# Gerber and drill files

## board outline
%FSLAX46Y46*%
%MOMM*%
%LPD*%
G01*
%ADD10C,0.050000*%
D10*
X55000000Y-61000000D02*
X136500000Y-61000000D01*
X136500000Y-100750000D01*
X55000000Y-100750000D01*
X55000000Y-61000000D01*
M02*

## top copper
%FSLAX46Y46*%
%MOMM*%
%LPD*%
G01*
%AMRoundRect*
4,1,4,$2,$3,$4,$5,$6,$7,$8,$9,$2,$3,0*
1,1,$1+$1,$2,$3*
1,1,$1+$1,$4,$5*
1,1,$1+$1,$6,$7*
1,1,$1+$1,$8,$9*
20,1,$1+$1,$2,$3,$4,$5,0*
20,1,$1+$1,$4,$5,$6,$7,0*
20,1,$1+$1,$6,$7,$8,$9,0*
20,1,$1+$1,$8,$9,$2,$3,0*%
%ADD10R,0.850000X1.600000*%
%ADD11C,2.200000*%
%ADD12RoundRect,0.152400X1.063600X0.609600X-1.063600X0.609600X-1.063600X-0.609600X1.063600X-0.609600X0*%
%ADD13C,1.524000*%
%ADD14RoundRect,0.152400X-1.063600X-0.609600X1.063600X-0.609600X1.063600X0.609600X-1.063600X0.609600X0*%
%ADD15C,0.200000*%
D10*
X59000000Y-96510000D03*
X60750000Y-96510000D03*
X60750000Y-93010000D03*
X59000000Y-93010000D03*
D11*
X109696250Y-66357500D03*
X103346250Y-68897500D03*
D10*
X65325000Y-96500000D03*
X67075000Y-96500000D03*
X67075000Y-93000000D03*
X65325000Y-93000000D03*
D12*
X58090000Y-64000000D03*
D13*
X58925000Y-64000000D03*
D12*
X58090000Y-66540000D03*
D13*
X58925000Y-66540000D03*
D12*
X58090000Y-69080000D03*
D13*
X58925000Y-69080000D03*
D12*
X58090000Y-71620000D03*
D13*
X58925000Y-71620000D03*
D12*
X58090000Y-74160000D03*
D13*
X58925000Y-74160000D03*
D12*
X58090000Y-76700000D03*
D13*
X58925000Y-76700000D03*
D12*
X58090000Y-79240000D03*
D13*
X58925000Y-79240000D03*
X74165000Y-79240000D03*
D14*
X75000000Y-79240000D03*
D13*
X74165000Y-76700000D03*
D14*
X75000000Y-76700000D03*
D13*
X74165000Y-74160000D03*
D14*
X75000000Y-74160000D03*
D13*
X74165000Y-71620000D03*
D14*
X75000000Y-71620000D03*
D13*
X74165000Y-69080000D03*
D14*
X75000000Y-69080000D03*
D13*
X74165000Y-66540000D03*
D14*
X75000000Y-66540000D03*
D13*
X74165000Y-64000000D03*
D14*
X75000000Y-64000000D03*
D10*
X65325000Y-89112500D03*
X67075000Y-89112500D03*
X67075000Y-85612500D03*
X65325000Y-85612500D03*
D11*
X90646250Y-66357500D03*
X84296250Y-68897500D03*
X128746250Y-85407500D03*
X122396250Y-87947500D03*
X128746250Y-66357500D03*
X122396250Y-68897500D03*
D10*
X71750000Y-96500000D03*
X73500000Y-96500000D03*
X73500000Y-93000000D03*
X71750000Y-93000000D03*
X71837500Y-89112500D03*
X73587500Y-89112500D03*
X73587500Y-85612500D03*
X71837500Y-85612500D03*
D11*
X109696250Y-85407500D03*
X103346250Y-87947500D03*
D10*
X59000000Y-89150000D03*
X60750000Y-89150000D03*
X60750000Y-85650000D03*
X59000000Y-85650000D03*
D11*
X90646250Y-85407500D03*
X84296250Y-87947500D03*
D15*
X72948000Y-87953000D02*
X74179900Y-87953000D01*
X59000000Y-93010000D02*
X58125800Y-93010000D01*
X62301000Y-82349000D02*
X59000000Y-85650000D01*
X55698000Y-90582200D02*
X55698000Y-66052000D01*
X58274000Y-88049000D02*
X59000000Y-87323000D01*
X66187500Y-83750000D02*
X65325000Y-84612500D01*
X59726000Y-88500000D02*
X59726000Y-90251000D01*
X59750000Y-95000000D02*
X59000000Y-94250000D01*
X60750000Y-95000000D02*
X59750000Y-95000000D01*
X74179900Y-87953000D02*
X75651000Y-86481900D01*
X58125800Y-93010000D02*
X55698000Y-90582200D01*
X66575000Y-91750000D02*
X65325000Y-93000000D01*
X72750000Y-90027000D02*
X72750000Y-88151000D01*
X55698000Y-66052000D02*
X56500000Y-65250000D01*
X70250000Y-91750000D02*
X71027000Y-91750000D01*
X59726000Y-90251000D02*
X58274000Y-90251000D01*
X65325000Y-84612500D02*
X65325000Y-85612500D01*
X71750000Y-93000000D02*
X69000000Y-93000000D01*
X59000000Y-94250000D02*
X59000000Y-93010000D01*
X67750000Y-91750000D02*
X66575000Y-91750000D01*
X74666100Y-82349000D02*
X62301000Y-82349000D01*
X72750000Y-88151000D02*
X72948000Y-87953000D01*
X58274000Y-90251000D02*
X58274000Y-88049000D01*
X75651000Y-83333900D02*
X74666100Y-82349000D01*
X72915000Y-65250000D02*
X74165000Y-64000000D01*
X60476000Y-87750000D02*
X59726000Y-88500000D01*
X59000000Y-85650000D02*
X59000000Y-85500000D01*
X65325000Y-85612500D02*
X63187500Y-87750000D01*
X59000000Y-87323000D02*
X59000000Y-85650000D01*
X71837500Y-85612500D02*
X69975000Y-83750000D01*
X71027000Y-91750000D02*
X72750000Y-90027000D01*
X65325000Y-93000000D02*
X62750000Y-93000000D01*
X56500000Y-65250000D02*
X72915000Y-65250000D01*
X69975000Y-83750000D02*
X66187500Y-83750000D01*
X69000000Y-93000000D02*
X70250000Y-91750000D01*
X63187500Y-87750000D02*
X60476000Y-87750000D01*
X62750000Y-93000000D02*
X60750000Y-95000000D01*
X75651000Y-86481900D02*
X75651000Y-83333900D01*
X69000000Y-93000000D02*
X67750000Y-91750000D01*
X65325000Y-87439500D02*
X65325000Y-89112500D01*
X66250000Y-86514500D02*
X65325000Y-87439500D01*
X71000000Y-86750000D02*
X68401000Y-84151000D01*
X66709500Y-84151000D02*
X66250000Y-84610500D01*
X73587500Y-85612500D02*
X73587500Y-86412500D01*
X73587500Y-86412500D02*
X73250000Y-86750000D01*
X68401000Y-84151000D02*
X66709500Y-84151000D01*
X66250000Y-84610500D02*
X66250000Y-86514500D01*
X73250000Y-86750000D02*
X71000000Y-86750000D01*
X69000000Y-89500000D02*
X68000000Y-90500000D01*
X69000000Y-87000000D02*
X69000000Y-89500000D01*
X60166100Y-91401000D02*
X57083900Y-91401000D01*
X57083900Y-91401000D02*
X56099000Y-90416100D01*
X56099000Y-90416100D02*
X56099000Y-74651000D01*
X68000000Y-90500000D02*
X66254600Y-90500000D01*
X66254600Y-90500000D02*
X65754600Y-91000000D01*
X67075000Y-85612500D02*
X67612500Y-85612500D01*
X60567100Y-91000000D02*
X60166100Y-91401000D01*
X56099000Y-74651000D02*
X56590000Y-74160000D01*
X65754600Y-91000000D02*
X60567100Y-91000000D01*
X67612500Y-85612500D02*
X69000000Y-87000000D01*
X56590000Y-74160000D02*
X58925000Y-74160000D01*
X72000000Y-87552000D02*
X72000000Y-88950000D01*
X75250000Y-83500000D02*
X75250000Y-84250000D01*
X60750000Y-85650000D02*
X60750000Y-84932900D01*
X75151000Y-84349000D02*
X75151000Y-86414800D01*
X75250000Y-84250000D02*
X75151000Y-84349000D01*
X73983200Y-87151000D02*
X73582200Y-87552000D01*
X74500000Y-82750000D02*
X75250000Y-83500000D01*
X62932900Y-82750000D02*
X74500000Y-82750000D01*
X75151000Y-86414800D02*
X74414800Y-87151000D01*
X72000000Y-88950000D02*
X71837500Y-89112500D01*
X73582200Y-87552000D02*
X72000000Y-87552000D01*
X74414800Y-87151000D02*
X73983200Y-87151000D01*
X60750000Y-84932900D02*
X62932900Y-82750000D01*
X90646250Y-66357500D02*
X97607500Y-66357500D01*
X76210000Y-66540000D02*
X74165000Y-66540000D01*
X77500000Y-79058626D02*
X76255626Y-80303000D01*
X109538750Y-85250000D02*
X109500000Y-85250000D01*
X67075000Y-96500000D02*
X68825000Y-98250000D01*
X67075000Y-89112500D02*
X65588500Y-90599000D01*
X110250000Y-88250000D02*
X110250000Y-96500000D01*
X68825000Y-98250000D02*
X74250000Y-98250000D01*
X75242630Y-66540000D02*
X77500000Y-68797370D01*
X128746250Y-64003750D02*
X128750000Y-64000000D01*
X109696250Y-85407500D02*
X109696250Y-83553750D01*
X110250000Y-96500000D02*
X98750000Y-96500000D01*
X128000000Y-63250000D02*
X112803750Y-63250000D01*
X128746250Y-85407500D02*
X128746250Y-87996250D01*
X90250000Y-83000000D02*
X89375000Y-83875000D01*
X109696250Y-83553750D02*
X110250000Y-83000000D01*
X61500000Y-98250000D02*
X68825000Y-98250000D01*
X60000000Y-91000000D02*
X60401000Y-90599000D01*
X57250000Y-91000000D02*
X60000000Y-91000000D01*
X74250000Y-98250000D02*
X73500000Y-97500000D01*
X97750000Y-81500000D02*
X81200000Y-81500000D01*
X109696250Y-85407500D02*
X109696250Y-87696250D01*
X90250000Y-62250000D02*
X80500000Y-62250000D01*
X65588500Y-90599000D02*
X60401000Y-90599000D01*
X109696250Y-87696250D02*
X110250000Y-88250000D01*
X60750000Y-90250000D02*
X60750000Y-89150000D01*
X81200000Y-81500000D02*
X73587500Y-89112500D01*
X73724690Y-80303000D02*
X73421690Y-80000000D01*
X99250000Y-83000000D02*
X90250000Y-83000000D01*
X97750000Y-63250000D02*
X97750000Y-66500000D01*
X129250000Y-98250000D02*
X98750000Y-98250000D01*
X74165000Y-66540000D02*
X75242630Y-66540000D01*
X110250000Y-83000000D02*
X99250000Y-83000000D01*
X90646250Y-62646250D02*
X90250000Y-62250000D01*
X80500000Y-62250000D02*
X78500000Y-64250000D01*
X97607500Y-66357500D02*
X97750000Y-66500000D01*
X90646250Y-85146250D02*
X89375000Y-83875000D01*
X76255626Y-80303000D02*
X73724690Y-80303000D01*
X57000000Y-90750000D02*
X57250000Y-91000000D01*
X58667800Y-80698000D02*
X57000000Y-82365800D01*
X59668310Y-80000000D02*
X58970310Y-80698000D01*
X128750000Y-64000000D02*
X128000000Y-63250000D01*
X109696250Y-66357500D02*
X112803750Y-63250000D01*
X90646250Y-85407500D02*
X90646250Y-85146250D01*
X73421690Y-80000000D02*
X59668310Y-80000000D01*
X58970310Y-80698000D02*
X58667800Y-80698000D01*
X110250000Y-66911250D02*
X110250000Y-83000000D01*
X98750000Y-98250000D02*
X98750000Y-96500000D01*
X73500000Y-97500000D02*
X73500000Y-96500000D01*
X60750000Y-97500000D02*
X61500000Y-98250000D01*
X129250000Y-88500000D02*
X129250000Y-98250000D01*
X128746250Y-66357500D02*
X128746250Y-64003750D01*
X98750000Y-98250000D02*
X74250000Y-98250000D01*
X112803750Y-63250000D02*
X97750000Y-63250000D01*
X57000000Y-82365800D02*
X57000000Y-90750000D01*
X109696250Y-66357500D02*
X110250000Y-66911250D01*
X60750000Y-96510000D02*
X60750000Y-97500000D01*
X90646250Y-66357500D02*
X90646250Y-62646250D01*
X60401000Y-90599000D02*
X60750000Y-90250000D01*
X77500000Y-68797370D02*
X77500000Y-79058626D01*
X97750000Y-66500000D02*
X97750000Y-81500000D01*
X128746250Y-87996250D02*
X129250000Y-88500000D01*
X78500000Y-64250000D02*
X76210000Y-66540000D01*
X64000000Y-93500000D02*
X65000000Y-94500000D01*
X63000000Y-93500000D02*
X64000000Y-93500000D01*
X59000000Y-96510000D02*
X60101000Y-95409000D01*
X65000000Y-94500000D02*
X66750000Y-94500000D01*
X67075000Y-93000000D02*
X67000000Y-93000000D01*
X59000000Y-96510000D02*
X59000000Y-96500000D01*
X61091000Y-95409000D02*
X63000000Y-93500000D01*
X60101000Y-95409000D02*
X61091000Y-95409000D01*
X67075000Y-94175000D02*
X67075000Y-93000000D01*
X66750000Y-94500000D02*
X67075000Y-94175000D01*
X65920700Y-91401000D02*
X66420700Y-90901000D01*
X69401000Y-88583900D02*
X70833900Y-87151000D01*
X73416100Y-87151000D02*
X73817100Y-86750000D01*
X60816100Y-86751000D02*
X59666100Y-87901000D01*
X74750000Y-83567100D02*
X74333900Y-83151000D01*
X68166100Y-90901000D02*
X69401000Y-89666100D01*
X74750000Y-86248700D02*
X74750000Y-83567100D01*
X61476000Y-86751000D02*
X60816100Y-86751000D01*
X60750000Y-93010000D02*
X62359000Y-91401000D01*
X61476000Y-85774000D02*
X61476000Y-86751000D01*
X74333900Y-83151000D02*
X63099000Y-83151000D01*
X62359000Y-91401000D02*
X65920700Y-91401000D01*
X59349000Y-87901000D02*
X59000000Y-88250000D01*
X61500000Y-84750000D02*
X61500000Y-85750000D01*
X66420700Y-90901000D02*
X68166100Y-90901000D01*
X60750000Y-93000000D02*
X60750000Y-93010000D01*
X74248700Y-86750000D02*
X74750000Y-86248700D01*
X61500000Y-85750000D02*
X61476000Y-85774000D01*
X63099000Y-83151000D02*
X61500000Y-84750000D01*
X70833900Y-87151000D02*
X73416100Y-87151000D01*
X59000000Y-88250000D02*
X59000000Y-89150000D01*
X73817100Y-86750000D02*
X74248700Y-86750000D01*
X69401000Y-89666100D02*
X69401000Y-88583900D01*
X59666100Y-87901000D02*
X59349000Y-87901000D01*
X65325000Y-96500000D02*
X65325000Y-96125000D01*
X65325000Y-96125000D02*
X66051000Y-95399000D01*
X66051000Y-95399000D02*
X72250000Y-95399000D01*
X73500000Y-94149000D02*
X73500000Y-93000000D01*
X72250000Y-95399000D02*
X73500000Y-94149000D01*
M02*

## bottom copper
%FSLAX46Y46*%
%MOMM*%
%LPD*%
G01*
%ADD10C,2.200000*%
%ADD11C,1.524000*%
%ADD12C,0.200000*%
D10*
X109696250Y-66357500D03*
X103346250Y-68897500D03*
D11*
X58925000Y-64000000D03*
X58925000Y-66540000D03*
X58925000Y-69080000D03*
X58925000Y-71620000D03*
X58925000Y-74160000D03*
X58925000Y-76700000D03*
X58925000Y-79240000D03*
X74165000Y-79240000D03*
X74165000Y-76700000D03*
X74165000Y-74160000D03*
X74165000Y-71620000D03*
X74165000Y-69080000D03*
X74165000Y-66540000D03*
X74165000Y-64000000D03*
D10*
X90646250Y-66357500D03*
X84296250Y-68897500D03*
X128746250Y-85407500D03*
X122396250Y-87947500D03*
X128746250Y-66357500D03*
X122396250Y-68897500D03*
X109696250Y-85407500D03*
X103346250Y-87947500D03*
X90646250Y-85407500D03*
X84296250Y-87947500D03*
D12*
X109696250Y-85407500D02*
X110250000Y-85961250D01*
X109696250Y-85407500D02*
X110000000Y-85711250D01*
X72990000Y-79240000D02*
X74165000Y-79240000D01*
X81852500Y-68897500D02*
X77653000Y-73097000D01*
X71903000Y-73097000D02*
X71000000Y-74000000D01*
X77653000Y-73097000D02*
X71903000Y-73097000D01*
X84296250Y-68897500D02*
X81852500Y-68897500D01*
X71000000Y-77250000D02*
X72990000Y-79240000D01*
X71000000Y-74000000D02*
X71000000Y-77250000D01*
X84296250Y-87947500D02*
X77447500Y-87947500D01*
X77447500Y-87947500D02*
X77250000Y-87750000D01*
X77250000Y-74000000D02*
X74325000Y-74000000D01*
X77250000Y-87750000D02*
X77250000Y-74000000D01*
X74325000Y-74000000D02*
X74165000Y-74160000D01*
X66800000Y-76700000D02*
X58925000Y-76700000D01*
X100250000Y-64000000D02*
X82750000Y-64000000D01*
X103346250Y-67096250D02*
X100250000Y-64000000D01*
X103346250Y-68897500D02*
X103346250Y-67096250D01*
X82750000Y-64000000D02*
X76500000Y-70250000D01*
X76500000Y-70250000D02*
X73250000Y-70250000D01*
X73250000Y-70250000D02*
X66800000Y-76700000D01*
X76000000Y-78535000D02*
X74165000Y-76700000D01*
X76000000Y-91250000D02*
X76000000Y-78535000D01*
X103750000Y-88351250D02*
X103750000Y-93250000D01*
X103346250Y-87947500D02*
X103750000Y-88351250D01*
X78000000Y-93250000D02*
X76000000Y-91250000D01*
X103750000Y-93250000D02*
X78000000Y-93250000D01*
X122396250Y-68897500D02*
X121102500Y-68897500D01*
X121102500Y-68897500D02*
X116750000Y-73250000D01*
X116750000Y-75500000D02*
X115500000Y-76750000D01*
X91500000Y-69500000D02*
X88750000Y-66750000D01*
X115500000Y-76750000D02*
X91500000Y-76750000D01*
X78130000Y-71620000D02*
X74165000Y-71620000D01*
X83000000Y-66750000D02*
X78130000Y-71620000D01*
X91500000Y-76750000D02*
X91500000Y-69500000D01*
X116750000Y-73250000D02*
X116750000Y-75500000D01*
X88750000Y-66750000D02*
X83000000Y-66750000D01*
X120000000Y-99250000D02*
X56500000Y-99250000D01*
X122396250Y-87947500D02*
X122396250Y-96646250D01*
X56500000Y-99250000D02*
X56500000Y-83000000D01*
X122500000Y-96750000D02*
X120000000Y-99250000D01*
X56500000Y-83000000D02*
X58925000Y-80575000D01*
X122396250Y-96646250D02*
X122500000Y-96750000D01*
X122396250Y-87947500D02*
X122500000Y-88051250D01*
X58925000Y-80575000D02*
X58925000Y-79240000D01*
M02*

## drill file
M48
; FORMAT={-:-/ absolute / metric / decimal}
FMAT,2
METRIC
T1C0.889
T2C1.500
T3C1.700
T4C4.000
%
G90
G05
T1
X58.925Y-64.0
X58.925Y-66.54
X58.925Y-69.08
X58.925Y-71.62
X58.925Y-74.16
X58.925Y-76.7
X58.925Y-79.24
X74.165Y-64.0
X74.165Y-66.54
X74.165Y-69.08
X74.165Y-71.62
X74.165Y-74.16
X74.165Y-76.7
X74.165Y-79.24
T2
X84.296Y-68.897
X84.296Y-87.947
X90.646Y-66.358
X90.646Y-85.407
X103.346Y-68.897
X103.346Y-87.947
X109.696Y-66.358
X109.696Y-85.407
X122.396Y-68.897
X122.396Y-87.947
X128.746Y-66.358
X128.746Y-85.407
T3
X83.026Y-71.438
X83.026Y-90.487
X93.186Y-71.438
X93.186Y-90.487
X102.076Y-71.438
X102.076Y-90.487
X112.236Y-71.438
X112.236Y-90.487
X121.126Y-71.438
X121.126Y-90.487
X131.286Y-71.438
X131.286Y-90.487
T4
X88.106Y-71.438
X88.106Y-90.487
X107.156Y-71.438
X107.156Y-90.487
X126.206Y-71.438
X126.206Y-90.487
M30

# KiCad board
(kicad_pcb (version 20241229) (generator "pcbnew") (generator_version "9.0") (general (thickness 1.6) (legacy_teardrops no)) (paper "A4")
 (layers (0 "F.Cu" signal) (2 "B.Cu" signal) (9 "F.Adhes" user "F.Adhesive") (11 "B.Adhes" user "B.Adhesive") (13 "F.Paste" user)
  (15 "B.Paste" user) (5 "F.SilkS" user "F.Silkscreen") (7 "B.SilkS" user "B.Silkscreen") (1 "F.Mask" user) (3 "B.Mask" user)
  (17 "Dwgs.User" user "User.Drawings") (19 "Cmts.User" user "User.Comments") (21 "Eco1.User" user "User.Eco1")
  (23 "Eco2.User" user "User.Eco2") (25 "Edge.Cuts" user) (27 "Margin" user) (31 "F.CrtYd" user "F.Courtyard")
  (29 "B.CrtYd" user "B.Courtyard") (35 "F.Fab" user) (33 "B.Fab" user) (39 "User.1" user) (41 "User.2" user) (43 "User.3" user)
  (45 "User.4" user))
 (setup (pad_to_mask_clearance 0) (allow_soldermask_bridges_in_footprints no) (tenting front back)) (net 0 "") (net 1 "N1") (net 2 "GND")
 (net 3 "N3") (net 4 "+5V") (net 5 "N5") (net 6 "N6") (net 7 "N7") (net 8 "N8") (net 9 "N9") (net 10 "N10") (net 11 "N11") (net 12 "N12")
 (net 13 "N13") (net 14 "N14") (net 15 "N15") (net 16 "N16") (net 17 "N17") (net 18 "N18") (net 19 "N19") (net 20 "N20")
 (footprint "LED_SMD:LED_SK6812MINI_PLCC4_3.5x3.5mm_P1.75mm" (layer "F.Cu") (at 59.875 94.76 90)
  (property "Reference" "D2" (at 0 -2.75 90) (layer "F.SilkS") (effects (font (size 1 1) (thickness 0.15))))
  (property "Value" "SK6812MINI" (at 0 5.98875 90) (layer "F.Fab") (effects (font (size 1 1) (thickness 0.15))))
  (pad "1" smd rect (at -1.75 -0.875 90) (size 1.6 0.85) (layers "F.Cu" "F.Mask" "F.Paste") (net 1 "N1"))
  (pad "2" smd rect (at -1.75 0.875 90) (size 1.6 0.85) (layers "F.Cu" "F.Mask" "F.Paste") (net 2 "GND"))
  (pad "3" smd rect (at 1.75 0.875 90) (size 1.6 0.85) (layers "F.Cu" "F.Mask" "F.Paste") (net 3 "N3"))
  (pad "4" smd rect (at 1.75 -0.875 90) (size 1.6 0.85) (layers "F.Cu" "F.Mask" "F.Paste") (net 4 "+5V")))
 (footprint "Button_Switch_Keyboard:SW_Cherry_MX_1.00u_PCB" (layer "F.Cu") (at 109.69625 66.3575)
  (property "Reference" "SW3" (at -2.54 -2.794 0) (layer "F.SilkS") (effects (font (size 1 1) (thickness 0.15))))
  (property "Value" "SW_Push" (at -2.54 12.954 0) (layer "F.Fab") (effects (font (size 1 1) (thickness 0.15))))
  (pad "" np_thru_hole circle (at -7.62 5.08) (size 1.7 1.7) (drill 1.7) (layers "*.Cu" "*.Mask"))
  (pad "" np_thru_hole circle (at -2.54 5.08) (size 4 4) (drill 4) (layers "*.Cu" "*.Mask"))
  (pad "" np_thru_hole circle (at 2.54 5.08) (size 1.7 1.7) (drill 1.7) (layers "*.Cu" "*.Mask"))
  (pad "1" thru_hole circle (at 0 0) (size 2.2 2.2) (drill 1.5) (layers "*.Cu" "*.Mask") (remove_unused_layers no) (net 2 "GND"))
  (pad "2" thru_hole circle (at -6.35 2.54) (size 2.2 2.2) (drill 1.5) (layers "*.Cu" "*.Mask") (remove_unused_layers no) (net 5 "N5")))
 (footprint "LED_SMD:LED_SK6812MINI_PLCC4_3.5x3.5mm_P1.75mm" (layer "F.Cu") (at 66.2 94.75 90)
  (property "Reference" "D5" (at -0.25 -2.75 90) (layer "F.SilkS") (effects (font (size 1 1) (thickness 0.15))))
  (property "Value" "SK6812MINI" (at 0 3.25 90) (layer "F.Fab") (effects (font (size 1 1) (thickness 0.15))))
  (pad "1" smd rect (at -1.75 -0.875 90) (size 1.6 0.85) (layers "F.Cu" "F.Mask" "F.Paste") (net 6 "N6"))
  (pad "2" smd rect (at -1.75 0.875 90) (size 1.6 0.85) (layers "F.Cu" "F.Mask" "F.Paste") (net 2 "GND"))
  (pad "3" smd rect (at 1.75 0.875 90) (size 1.6 0.85) (layers "F.Cu" "F.Mask" "F.Paste") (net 1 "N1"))
  (pad "4" smd rect (at 1.75 -0.875 90) (size 1.6 0.85) (layers "F.Cu" "F.Mask" "F.Paste") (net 4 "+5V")))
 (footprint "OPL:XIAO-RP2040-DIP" (layer "F.Cu") (at 66.545 71.62)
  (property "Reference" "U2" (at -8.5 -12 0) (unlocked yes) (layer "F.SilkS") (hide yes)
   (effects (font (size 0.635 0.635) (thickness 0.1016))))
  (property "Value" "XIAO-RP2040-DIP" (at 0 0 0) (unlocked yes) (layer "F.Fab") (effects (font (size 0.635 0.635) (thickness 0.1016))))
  (pad "1" smd roundrect (at -8.455 -7.62 180) (size 2.432 1.524) (layers "F.Cu" "F.Mask") (roundrect_rratio 0.1) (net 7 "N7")
   (thermal_bridge_angle 45))
  (pad "1" thru_hole circle (at -7.62 -7.62 180) (size 1.524 1.524) (drill 0.889) (layers "*.Cu" "*.Mask") (remove_unused_layers no)
   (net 7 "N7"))
  (pad "2" smd roundrect (at -8.455 -5.08 180) (size 2.432 1.524) (layers "F.Cu" "F.Mask") (roundrect_rratio 0.1) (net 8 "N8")
   (thermal_bridge_angle 45))
  (pad "2" thru_hole circle (at -7.62 -5.08 180) (size 1.524 1.524) (drill 0.889) (layers "*.Cu" "*.Mask") (remove_unused_layers no)
   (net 8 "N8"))
  (pad "3" smd roundrect (at -8.455 -2.54 180) (size 2.432 1.524) (layers "F.Cu" "F.Mask") (roundrect_rratio 0.1) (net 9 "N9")
   (thermal_bridge_angle 45))
  (pad "3" thru_hole circle (at -7.62 -2.54 180) (size 1.524 1.524) (drill 0.889) (layers "*.Cu" "*.Mask") (remove_unused_layers no)
   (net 9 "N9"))
  (pad "4" smd roundrect (at -8.455 0 180) (size 2.432 1.524) (layers "F.Cu" "F.Mask") (roundrect_rratio 0.1) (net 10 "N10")
   (thermal_bridge_angle 45))
  (pad "4" thru_hole circle (at -7.62 0 180) (size 1.524 1.524) (drill 0.889) (layers "*.Cu" "*.Mask") (remove_unused_layers no)
   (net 10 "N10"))
  (pad "5" smd roundrect (at -8.455 2.54 180) (size 2.432 1.524) (layers "F.Cu" "F.Mask") (roundrect_rratio 0.1) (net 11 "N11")
   (thermal_bridge_angle 45))
  (pad "5" thru_hole circle (at -7.62 2.54 180) (size 1.524 1.524) (drill 0.889) (layers "*.Cu" "*.Mask") (remove_unused_layers no)
   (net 11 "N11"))
  (pad "6" smd roundrect (at -8.455 5.08 180) (size 2.432 1.524) (layers "F.Cu" "F.Mask") (roundrect_rratio 0.1) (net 5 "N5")
   (thermal_bridge_angle 45))
  (pad "6" thru_hole circle (at -7.62 5.08 180) (size 1.524 1.524) (drill 0.889) (layers "*.Cu" "*.Mask") (remove_unused_layers no)
   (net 5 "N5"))
  (pad "7" smd roundrect (at -8.455 7.62 180) (size 2.432 1.524) (layers "F.Cu" "F.Mask") (roundrect_rratio 0.1) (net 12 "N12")
   (thermal_bridge_angle 45))
  (pad "7" thru_hole circle (at -7.62 7.62 180) (size 1.524 1.524) (drill 0.889) (layers "*.Cu" "*.Mask") (remove_unused_layers no)
   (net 12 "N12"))
  (pad "8" thru_hole circle (at 7.62 7.62) (size 1.524 1.524) (drill 0.889) (layers "*.Cu" "*.Mask") (remove_unused_layers no)
   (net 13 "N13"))
  (pad "8" smd roundrect (at 8.455 7.62) (size 2.432 1.524) (layers "F.Cu" "F.Mask") (roundrect_rratio 0.1) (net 13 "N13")
   (thermal_bridge_angle 45))
  (pad "9" thru_hole circle (at 7.62 5.08) (size 1.524 1.524) (drill 0.889) (layers "*.Cu" "*.Mask") (remove_unused_layers no)
   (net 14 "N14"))
  (pad "9" smd roundrect (at 8.455 5.08) (size 2.432 1.524) (layers "F.Cu" "F.Mask") (roundrect_rratio 0.1) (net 14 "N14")
   (thermal_bridge_angle 45))
  (pad "10" thru_hole circle (at 7.62 2.54) (size 1.524 1.524) (drill 0.889) (layers "*.Cu" "*.Mask") (remove_unused_layers no)
   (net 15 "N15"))
  (pad "10" smd roundrect (at 8.455 2.54) (size 2.432 1.524) (layers "F.Cu" "F.Mask") (roundrect_rratio 0.1) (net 15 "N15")
   (thermal_bridge_angle 45))
  (pad "11" thru_hole circle (at 7.62 0) (size 1.524 1.524) (drill 0.889) (layers "*.Cu" "*.Mask") (remove_unused_layers no) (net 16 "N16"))
  (pad "11" smd roundrect (at 8.455 0) (size 2.432 1.524) (layers "F.Cu" "F.Mask") (roundrect_rratio 0.1) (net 16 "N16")
   (thermal_bridge_angle 45))
  (pad "12" thru_hole circle (at 7.62 -2.54) (size 1.524 1.524) (drill 0.889) (layers "*.Cu" "*.Mask") (remove_unused_layers no)
   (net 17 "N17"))
  (pad "12" smd roundrect (at 8.455 -2.54) (size 2.432 1.524) (layers "F.Cu" "F.Mask") (roundrect_rratio 0.1) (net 17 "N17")
   (thermal_bridge_angle 45))
  (pad "13" thru_hole circle (at 7.62 -5.08) (size 1.524 1.524) (drill 0.889) (layers "*.Cu" "*.Mask") (remove_unused_layers no)
   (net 2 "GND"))
  (pad "13" smd roundrect (at 8.455 -5.08) (size 2.432 1.524) (layers "F.Cu" "F.Mask") (roundrect_rratio 0.1) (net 2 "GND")
   (thermal_bridge_angle 45))
  (pad "14" thru_hole circle (at 7.62 -7.62) (size 1.524 1.524) (drill 0.889) (layers "*.Cu" "*.Mask") (remove_unused_layers no)
   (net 4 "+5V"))
  (pad "14" smd roundrect (at 8.455 -7.62) (size 2.432 1.524) (layers "F.Cu" "F.Mask") (roundrect_rratio 0.1) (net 4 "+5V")
   (thermal_bridge_angle 45)))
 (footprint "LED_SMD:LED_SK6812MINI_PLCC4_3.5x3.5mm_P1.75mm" (layer "F.Cu") (at 66.2 87.3625 90)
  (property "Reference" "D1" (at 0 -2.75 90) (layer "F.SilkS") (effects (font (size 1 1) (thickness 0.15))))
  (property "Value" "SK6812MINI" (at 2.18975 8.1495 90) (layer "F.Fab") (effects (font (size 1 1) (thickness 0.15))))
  (pad "1" smd rect (at -1.75 -0.875 90) (size 1.6 0.85) (layers "F.Cu" "F.Mask" "F.Paste") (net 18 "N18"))
  (pad "2" smd rect (at -1.75 0.875 90) (size 1.6 0.85) (layers "F.Cu" "F.Mask" "F.Paste") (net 2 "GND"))
  (pad "3" smd rect (at 1.75 0.875 90) (size 1.6 0.85) (layers "F.Cu" "F.Mask" "F.Paste") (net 11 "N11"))
  (pad "4" smd rect (at 1.75 -0.875 90) (size 1.6 0.85) (layers "F.Cu" "F.Mask" "F.Paste") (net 4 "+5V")))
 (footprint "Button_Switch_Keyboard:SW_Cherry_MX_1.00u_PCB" (layer "F.Cu") (at 90.64625 66.3575)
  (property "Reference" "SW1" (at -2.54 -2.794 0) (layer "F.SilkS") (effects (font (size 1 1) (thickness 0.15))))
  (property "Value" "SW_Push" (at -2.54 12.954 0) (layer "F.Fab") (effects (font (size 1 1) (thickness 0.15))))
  (pad "" np_thru_hole circle (at -7.62 5.08) (size 1.7 1.7) (drill 1.7) (layers "*.Cu" "*.Mask"))
  (pad "" np_thru_hole circle (at -2.54 5.08) (size 4 4) (drill 4) (layers "*.Cu" "*.Mask"))
  (pad "" np_thru_hole circle (at 2.54 5.08) (size 1.7 1.7) (drill 1.7) (layers "*.Cu" "*.Mask"))
  (pad "1" thru_hole circle (at 0 0) (size 2.2 2.2) (drill 1.5) (layers "*.Cu" "*.Mask") (remove_unused_layers no) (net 2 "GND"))
  (pad "2" thru_hole circle (at -6.35 2.54) (size 2.2 2.2) (drill 1.5) (layers "*.Cu" "*.Mask") (remove_unused_layers no) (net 13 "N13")))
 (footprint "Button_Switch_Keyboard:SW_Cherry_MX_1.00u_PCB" (layer "F.Cu") (at 128.74625 85.4075)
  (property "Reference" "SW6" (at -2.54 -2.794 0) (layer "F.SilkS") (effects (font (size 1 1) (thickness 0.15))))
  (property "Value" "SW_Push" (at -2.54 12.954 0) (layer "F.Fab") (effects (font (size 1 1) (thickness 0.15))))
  (pad "" np_thru_hole circle (at -7.62 5.08) (size 1.7 1.7) (drill 1.7) (layers "*.Cu" "*.Mask"))
  (pad "" np_thru_hole circle (at -2.54 5.08) (size 4 4) (drill 4) (layers "*.Cu" "*.Mask"))
  (pad "" np_thru_hole circle (at 2.54 5.08) (size 1.7 1.7) (drill 1.7) (layers "*.Cu" "*.Mask"))
  (pad "1" thru_hole circle (at 0 0) (size 2.2 2.2) (drill 1.5) (layers "*.Cu" "*.Mask") (remove_unused_layers no) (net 2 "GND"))
  (pad "2" thru_hole circle (at -6.35 2.54) (size 2.2 2.2) (drill 1.5) (layers "*.Cu" "*.Mask") (remove_unused_layers no) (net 12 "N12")))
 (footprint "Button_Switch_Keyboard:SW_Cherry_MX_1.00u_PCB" (layer "F.Cu") (at 128.74625 66.3575)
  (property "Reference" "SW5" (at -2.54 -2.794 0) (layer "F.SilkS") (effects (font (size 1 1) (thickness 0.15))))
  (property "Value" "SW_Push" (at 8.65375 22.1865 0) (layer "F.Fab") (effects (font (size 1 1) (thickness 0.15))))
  (pad "" np_thru_hole circle (at -7.62 5.08) (size 1.7 1.7) (drill 1.7) (layers "*.Cu" "*.Mask"))
  (pad "" np_thru_hole circle (at -2.54 5.08) (size 4 4) (drill 4) (layers "*.Cu" "*.Mask"))
  (pad "" np_thru_hole circle (at 2.54 5.08) (size 1.7 1.7) (drill 1.7) (layers "*.Cu" "*.Mask"))
  (pad "1" thru_hole circle (at 0 0) (size 2.2 2.2) (drill 1.5) (layers "*.Cu" "*.Mask") (remove_unused_layers no) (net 2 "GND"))
  (pad "2" thru_hole circle (at -6.35 2.54) (size 2.2 2.2) (drill 1.5) (layers "*.Cu" "*.Mask") (remove_unused_layers no) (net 16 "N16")))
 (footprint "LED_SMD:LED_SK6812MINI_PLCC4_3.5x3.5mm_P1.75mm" (layer "F.Cu") (at 72.625 94.75 90)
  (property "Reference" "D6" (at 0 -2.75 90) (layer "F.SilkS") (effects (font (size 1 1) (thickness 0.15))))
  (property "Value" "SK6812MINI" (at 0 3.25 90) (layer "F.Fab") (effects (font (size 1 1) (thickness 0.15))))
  (pad "1" smd rect (at -1.75 -0.875 90) (size 1.6 0.85) (layers "F.Cu" "F.Mask" "F.Paste") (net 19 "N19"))
  (pad "2" smd rect (at -1.75 0.875 90) (size 1.6 0.85) (layers "F.Cu" "F.Mask" "F.Paste") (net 2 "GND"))
  (pad "3" smd rect (at 1.75 0.875 90) (size 1.6 0.85) (layers "F.Cu" "F.Mask" "F.Paste") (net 6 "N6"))
  (pad "4" smd rect (at 1.75 -0.875 90) (size 1.6 0.85) (layers "F.Cu" "F.Mask" "F.Paste") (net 4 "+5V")))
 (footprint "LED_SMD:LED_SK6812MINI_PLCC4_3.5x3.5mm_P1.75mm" (layer "F.Cu") (at 72.7125 87.3625 90)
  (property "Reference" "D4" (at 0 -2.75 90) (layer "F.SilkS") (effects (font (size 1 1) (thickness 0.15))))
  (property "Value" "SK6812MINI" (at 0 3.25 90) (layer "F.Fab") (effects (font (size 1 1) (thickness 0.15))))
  (pad "1" smd rect (at -1.75 -0.875 90) (size 1.6 0.85) (layers "F.Cu" "F.Mask" "F.Paste") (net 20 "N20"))
  (pad "2" smd rect (at -1.75 0.875 90) (size 1.6 0.85) (layers "F.Cu" "F.Mask" "F.Paste") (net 2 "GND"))
  (pad "3" smd rect (at 1.75 0.875 90) (size 1.6 0.85) (layers "F.Cu" "F.Mask" "F.Paste") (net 18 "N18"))
  (pad "4" smd rect (at 1.75 -0.875 90) (size 1.6 0.85) (layers "F.Cu" "F.Mask" "F.Paste") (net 4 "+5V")))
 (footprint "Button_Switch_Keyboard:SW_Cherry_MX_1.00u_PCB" (layer "F.Cu") (at 109.69625 85.4075)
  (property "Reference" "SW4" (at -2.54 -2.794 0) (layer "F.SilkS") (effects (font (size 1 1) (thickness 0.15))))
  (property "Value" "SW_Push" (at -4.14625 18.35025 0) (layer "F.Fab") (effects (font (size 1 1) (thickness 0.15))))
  (pad "" np_thru_hole circle (at -7.62 5.08) (size 1.7 1.7) (drill 1.7) (layers "*.Cu" "*.Mask"))
  (pad "" np_thru_hole circle (at -2.54 5.08) (size 4 4) (drill 4) (layers "*.Cu" "*.Mask"))
  (pad "" np_thru_hole circle (at 2.54 5.08) (size 1.7 1.7) (drill 1.7) (layers "*.Cu" "*.Mask"))
  (pad "1" thru_hole circle (at 0 0) (size 2.2 2.2) (drill 1.5) (layers "*.Cu" "*.Mask") (remove_unused_layers no) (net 2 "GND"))
  (pad "2" thru_hole circle (at -6.35 2.54) (size 2.2 2.2) (drill 1.5) (layers "*.Cu" "*.Mask") (remove_unused_layers no) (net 14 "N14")))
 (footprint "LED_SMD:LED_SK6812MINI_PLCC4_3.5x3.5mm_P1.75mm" (layer "F.Cu") (at 59.875 87.4 90)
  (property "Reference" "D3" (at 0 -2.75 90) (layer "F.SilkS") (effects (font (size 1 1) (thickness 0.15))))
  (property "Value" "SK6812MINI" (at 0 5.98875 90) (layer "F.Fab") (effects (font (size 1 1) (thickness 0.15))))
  (pad "1" smd rect (at -1.75 -0.875 90) (size 1.6 0.85) (layers "F.Cu" "F.Mask" "F.Paste") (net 3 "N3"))
  (pad "2" smd rect (at -1.75 0.875 90) (size 1.6 0.85) (layers "F.Cu" "F.Mask" "F.Paste") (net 2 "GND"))
  (pad "3" smd rect (at 1.75 0.875 90) (size 1.6 0.85) (layers "F.Cu" "F.Mask" "F.Paste") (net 20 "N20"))
  (pad "4" smd rect (at 1.75 -0.875 90) (size 1.6 0.85) (layers "F.Cu" "F.Mask" "F.Paste") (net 4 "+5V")))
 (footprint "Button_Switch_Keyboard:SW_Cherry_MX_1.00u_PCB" (layer "F.Cu") (at 90.64625 85.4075)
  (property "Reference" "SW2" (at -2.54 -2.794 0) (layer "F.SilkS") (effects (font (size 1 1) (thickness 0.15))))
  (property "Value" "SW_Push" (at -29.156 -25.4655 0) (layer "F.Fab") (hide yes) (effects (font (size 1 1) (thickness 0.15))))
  (pad "" np_thru_hole circle (at -7.62 5.08) (size 1.7 1.7) (drill 1.7) (layers "*.Cu" "*.Mask"))
  (pad "" np_thru_hole circle (at -2.54 5.08) (size 4 4) (drill 4) (layers "*.Cu" "*.Mask"))
  (pad "" np_thru_hole circle (at 2.54 5.08) (size 1.7 1.7) (drill 1.7) (layers "*.Cu" "*.Mask"))
  (pad "1" thru_hole circle (at 0 0) (size 2.2 2.2) (drill 1.5) (layers "*.Cu" "*.Mask") (remove_unused_layers no) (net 2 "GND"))
  (pad "2" thru_hole circle (at -6.35 2.54) (size 2.2 2.2) (drill 1.5) (layers "*.Cu" "*.Mask") (remove_unused_layers no) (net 15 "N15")))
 (gr_rect (start 55 61) (end 136.5 100.75) (stroke (width 0.05) (type default)) (fill no) (layer "Edge.Cuts"))
 (segment (start 72.948 87.953) (end 74.1799 87.953) (width 0.2) (layer "F.Cu") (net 4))
 (segment (start 59 93.01) (end 58.1258 93.01) (width 0.2) (layer "F.Cu") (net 4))
 (segment (start 62.301 82.349) (end 59 85.65) (width 0.2) (layer "F.Cu") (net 4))
 (segment (start 55.698 90.5822) (end 55.698 66.052) (width 0.2) (layer "F.Cu") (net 4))
 (segment (start 58.274 88.049) (end 59 87.323) (width 0.2) (layer "F.Cu") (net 4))
 (segment (start 66.1875 83.75) (end 65.325 84.6125) (width 0.2) (layer "F.Cu") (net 4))
 (segment (start 59.726 88.5) (end 59.726 90.251) (width 0.2) (layer "F.Cu") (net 4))
 (segment (start 59.75 95) (end 59 94.25) (width 0.2) (layer "F.Cu") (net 4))
 (segment (start 60.75 95) (end 59.75 95) (width 0.2) (layer "F.Cu") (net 4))
 (segment (start 74.1799 87.953) (end 75.651 86.4819) (width 0.2) (layer "F.Cu") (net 4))
 (segment (start 58.1258 93.01) (end 55.698 90.5822) (width 0.2) (layer "F.Cu") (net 4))
 (segment (start 66.575 91.75) (end 65.325 93) (width 0.2) (layer "F.Cu") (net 4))
 (segment (start 72.75 90.027) (end 72.75 88.151) (width 0.2) (layer "F.Cu") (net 4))
 (segment (start 55.698 66.052) (end 56.5 65.25) (width 0.2) (layer "F.Cu") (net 4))
 (segment (start 70.25 91.75) (end 71.027 91.75) (width 0.2) (layer "F.Cu") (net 4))
 (segment (start 59.726 90.251) (end 58.274 90.251) (width 0.2) (layer "F.Cu") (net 4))
 (segment (start 65.325 84.6125) (end 65.325 85.6125) (width 0.2) (layer "F.Cu") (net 4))
 (segment (start 71.75 93) (end 69 93) (width 0.2) (layer "F.Cu") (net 4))
 (segment (start 59 94.25) (end 59 93.01) (width 0.2) (layer "F.Cu") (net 4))
 (segment (start 67.75 91.75) (end 66.575 91.75) (width 0.2) (layer "F.Cu") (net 4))
 (segment (start 74.6661 82.349) (end 62.301 82.349) (width 0.2) (layer "F.Cu") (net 4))
 (segment (start 72.75 88.151) (end 72.948 87.953) (width 0.2) (layer "F.Cu") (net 4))
 (segment (start 58.274 90.251) (end 58.274 88.049) (width 0.2) (layer "F.Cu") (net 4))
 (segment (start 75.651 83.3339) (end 74.6661 82.349) (width 0.2) (layer "F.Cu") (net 4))
 (segment (start 72.915 65.25) (end 74.165 64) (width 0.2) (layer "F.Cu") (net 4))
 (segment (start 60.476 87.75) (end 59.726 88.5) (width 0.2) (layer "F.Cu") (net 4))
 (segment (start 59 85.65) (end 59 85.5) (width 0.2) (layer "F.Cu") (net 4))
 (segment (start 65.325 85.6125) (end 63.1875 87.75) (width 0.2) (layer "F.Cu") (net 4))
 (segment (start 59 87.323) (end 59 85.65) (width 0.2) (layer "F.Cu") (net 4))
 (segment (start 71.8375 85.6125) (end 69.975 83.75) (width 0.2) (layer "F.Cu") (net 4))
 (segment (start 71.027 91.75) (end 72.75 90.027) (width 0.2) (layer "F.Cu") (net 4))
 (segment (start 65.325 93) (end 62.75 93) (width 0.2) (layer "F.Cu") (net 4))
 (segment (start 56.5 65.25) (end 72.915 65.25) (width 0.2) (layer "F.Cu") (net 4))
 (segment (start 69.975 83.75) (end 66.1875 83.75) (width 0.2) (layer "F.Cu") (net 4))
 (segment (start 69 93) (end 70.25 91.75) (width 0.2) (layer "F.Cu") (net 4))
 (segment (start 63.1875 87.75) (end 60.476 87.75) (width 0.2) (layer "F.Cu") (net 4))
 (segment (start 62.75 93) (end 60.75 95) (width 0.2) (layer "F.Cu") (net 4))
 (segment (start 75.651 86.4819) (end 75.651 83.3339) (width 0.2) (layer "F.Cu") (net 4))
 (segment (start 69 93) (end 67.75 91.75) (width 0.2) (layer "F.Cu") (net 4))
 (segment (start 65.325 87.4395) (end 65.325 89.1125) (width 0.2) (layer "F.Cu") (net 18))
 (segment (start 66.25 86.5145) (end 65.325 87.4395) (width 0.2) (layer "F.Cu") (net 18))
 (segment (start 71 86.75) (end 68.401 84.151) (width 0.2) (layer "F.Cu") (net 18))
 (segment (start 66.7095 84.151) (end 66.25 84.6105) (width 0.2) (layer "F.Cu") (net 18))
 (segment (start 73.5875 85.6125) (end 73.5875 86.4125) (width 0.2) (layer "F.Cu") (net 18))
 (segment (start 73.5875 86.4125) (end 73.25 86.75) (width 0.2) (layer "F.Cu") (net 18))
 (segment (start 68.401 84.151) (end 66.7095 84.151) (width 0.2) (layer "F.Cu") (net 18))
 (segment (start 66.25 84.6105) (end 66.25 86.5145) (width 0.2) (layer "F.Cu") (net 18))
 (segment (start 73.25 86.75) (end 71 86.75) (width 0.2) (layer "F.Cu") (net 18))
 (segment (start 69 89.5) (end 68 90.5) (width 0.2) (layer "F.Cu") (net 11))
 (segment (start 69 87) (end 69 89.5) (width 0.2) (layer "F.Cu") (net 11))
 (segment (start 60.1661 91.401) (end 57.0839 91.401) (width 0.2) (layer "F.Cu") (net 11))
 (segment (start 57.0839 91.401) (end 56.099 90.4161) (width 0.2) (layer "F.Cu") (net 11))
 (segment (start 56.099 90.4161) (end 56.099 74.651) (width 0.2) (layer "F.Cu") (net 11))
 (segment (start 68 90.5) (end 66.2546 90.5) (width 0.2) (layer "F.Cu") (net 11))
 (segment (start 66.2546 90.5) (end 65.7546 91) (width 0.2) (layer "F.Cu") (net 11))
 (segment (start 67.075 85.6125) (end 67.6125 85.6125) (width 0.2) (layer "F.Cu") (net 11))
 (segment (start 60.5671 91) (end 60.1661 91.401) (width 0.2) (layer "F.Cu") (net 11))
 (segment (start 56.099 74.651) (end 56.59 74.16) (width 0.2) (layer "F.Cu") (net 11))
 (segment (start 65.7546 91) (end 60.5671 91) (width 0.2) (layer "F.Cu") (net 11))
 (segment (start 67.6125 85.6125) (end 69 87) (width 0.2) (layer "F.Cu") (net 11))
 (segment (start 56.59 74.16) (end 58.925 74.16) (width 0.2) (layer "F.Cu") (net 11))
 (segment (start 72 87.552) (end 72 88.95) (width 0.2) (layer "F.Cu") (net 20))
 (segment (start 75.25 83.5) (end 75.25 84.25) (width 0.2) (layer "F.Cu") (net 20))
 (segment (start 60.75 85.65) (end 60.75 84.9329) (width 0.2) (layer "F.Cu") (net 20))
 (segment (start 75.151 84.349) (end 75.151 86.4148) (width 0.2) (layer "F.Cu") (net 20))
 (segment (start 75.25 84.25) (end 75.151 84.349) (width 0.2) (layer "F.Cu") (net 20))
 (segment (start 73.9832 87.151) (end 73.5822 87.552) (width 0.2) (layer "F.Cu") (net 20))
 (segment (start 74.5 82.75) (end 75.25 83.5) (width 0.2) (layer "F.Cu") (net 20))
 (segment (start 62.9329 82.75) (end 74.5 82.75) (width 0.2) (layer "F.Cu") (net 20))
 (segment (start 75.151 86.4148) (end 74.4148 87.151) (width 0.2) (layer "F.Cu") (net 20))
 (segment (start 72 88.95) (end 71.8375 89.1125) (width 0.2) (layer "F.Cu") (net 20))
 (segment (start 73.5822 87.552) (end 72 87.552) (width 0.2) (layer "F.Cu") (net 20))
 (segment (start 74.4148 87.151) (end 73.9832 87.151) (width 0.2) (layer "F.Cu") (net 20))
 (segment (start 60.75 84.9329) (end 62.9329 82.75) (width 0.2) (layer "F.Cu") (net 20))
 (segment (start 90.64625 66.3575) (end 97.6075 66.3575) (width 0.2) (layer "F.Cu") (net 2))
 (segment (start 76.21 66.54) (end 74.165 66.54) (width 0.2) (layer "F.Cu") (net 2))
 (segment (start 77.5 79.058626) (end 76.255626 80.303) (width 0.2) (layer "F.Cu") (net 2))
 (segment (start 109.53875 85.25) (end 109.5 85.25) (width 0.2) (layer "F.Cu") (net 2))
 (segment (start 67.075 96.5) (end 68.825 98.25) (width 0.2) (layer "F.Cu") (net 2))
 (segment (start 67.075 89.1125) (end 65.5885 90.599) (width 0.2) (layer "F.Cu") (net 2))
 (segment (start 110.25 88.25) (end 110.25 96.5) (width 0.2) (layer "F.Cu") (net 2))
 (segment (start 68.825 98.25) (end 74.25 98.25) (width 0.2) (layer "F.Cu") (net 2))
 (segment (start 75.24263 66.54) (end 77.5 68.79737) (width 0.2) (layer "F.Cu") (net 2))
 (segment (start 128.74625 64.00375) (end 128.75 64) (width 0.2) (layer "F.Cu") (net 2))
 (segment (start 109.69625 85.4075) (end 109.69625 83.55375) (width 0.2) (layer "F.Cu") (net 2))
 (segment (start 110.25 96.5) (end 98.75 96.5) (width 0.2) (layer "F.Cu") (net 2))
 (segment (start 128 63.25) (end 112.80375 63.25) (width 0.2) (layer "F.Cu") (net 2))
 (segment (start 128.74625 85.4075) (end 128.74625 87.99625) (width 0.2) (layer "F.Cu") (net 2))
 (segment (start 90.25 83) (end 89.375 83.875) (width 0.2) (layer "F.Cu") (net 2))
 (segment (start 109.69625 83.55375) (end 110.25 83) (width 0.2) (layer "F.Cu") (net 2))
 (segment (start 61.5 98.25) (end 68.825 98.25) (width 0.2) (layer "F.Cu") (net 2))
 (segment (start 60 91) (end 60.401 90.599) (width 0.2) (layer "F.Cu") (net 2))
 (segment (start 57.25 91) (end 60 91) (width 0.2) (layer "F.Cu") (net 2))
 (segment (start 74.25 98.25) (end 73.5 97.5) (width 0.2) (layer "F.Cu") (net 2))
 (segment (start 97.75 81.5) (end 81.2 81.5) (width 0.2) (layer "F.Cu") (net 2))
 (segment (start 109.69625 85.4075) (end 109.69625 87.69625) (width 0.2) (layer "F.Cu") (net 2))
 (segment (start 90.25 62.25) (end 80.5 62.25) (width 0.2) (layer "F.Cu") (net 2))
 (segment (start 65.5885 90.599) (end 60.401 90.599) (width 0.2) (layer "F.Cu") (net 2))
 (segment (start 109.69625 87.69625) (end 110.25 88.25) (width 0.2) (layer "F.Cu") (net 2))
 (segment (start 60.75 90.25) (end 60.75 89.15) (width 0.2) (layer "F.Cu") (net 2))
 (segment (start 81.2 81.5) (end 73.5875 89.1125) (width 0.2) (layer "F.Cu") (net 2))
 (segment (start 73.72469 80.303) (end 73.42169 80) (width 0.2) (layer "F.Cu") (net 2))
 (segment (start 99.25 83) (end 90.25 83) (width 0.2) (layer "F.Cu") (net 2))
 (segment (start 97.75 63.25) (end 97.75 66.5) (width 0.2) (layer "F.Cu") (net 2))
 (segment (start 129.25 98.25) (end 98.75 98.25) (width 0.2) (layer "F.Cu") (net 2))
 (segment (start 74.165 66.54) (end 75.24263 66.54) (width 0.2) (layer "F.Cu") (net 2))
 (segment (start 110.25 83) (end 99.25 83) (width 0.2) (layer "F.Cu") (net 2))
 (segment (start 90.64625 62.64625) (end 90.25 62.25) (width 0.2) (layer "F.Cu") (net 2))
 (segment (start 80.5 62.25) (end 78.5 64.25) (width 0.2) (layer "F.Cu") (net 2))
 (segment (start 97.6075 66.3575) (end 97.75 66.5) (width 0.2) (layer "F.Cu") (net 2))
 (segment (start 90.64625 85.14625) (end 89.375 83.875) (width 0.2) (layer "F.Cu") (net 2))
 (segment (start 76.255626 80.303) (end 73.72469 80.303) (width 0.2) (layer "F.Cu") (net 2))
 (segment (start 57 90.75) (end 57.25 91) (width 0.2) (layer "F.Cu") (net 2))
 (segment (start 58.6678 80.698) (end 57 82.3658) (width 0.2) (layer "F.Cu") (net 2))
 (segment (start 59.66831 80) (end 58.97031 80.698) (width 0.2) (layer "F.Cu") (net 2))
 (segment (start 128.75 64) (end 128 63.25) (width 0.2) (layer "F.Cu") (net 2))
 (segment (start 109.69625 66.3575) (end 112.80375 63.25) (width 0.2) (layer "F.Cu") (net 2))
 (segment (start 90.64625 85.4075) (end 90.64625 85.14625) (width 0.2) (layer "F.Cu") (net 2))
 (segment (start 73.42169 80) (end 59.66831 80) (width 0.2) (layer "F.Cu") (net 2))
 (segment (start 58.97031 80.698) (end 58.6678 80.698) (width 0.2) (layer "F.Cu") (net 2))
 (segment (start 110.25 66.91125) (end 110.25 83) (width 0.2) (layer "F.Cu") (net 2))
 (segment (start 98.75 98.25) (end 98.75 96.5) (width 0.2) (layer "F.Cu") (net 2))
 (segment (start 73.5 97.5) (end 73.5 96.5) (width 0.2) (layer "F.Cu") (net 2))
 (segment (start 60.75 97.5) (end 61.5 98.25) (width 0.2) (layer "F.Cu") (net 2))
 (segment (start 129.25 88.5) (end 129.25 98.25) (width 0.2) (layer "F.Cu") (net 2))
 (segment (start 128.74625 66.3575) (end 128.74625 64.00375) (width 0.2) (layer "F.Cu") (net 2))
 (segment (start 98.75 98.25) (end 74.25 98.25) (width 0.2) (layer "F.Cu") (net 2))
 (segment (start 112.80375 63.25) (end 97.75 63.25) (width 0.2) (layer "F.Cu") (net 2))
 (segment (start 57 82.3658) (end 57 90.75) (width 0.2) (layer "F.Cu") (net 2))
 (segment (start 109.69625 66.3575) (end 110.25 66.91125) (width 0.2) (layer "F.Cu") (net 2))
 (segment (start 60.75 96.51) (end 60.75 97.5) (width 0.2) (layer "F.Cu") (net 2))
 (segment (start 90.64625 66.3575) (end 90.64625 62.64625) (width 0.2) (layer "F.Cu") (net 2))
 (segment (start 60.401 90.599) (end 60.75 90.25) (width 0.2) (layer "F.Cu") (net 2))
 (segment (start 77.5 68.79737) (end 77.5 79.058626) (width 0.2) (layer "F.Cu") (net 2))
 (segment (start 97.75 66.5) (end 97.75 81.5) (width 0.2) (layer "F.Cu") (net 2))
 (segment (start 128.74625 87.99625) (end 129.25 88.5) (width 0.2) (layer "F.Cu") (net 2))
 (segment (start 78.5 64.25) (end 76.21 66.54) (width 0.2) (layer "F.Cu") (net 2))
 (segment (start 109.69625 85.4075) (end 110.25 85.96125) (width 0.2) (layer "B.Cu") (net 2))
 (segment (start 109.69625 85.4075) (end 110 85.71125) (width 0.2) (layer "B.Cu") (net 2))
 (segment (start 72.99 79.24) (end 74.165 79.24) (width 0.2) (layer "B.Cu") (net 13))
 (segment (start 81.8525 68.8975) (end 77.653 73.097) (width 0.2) (layer "B.Cu") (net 13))
 (segment (start 71.903 73.097) (end 71 74) (width 0.2) (layer "B.Cu") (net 13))
 (segment (start 77.653 73.097) (end 71.903 73.097) (width 0.2) (layer "B.Cu") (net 13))
 (segment (start 84.29625 68.8975) (end 81.8525 68.8975) (width 0.2) (layer "B.Cu") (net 13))
 (segment (start 71 77.25) (end 72.99 79.24) (width 0.2) (layer "B.Cu") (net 13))
 (segment (start 71 74) (end 71 77.25) (width 0.2) (layer "B.Cu") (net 13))
 (segment (start 84.29625 87.9475) (end 77.4475 87.9475) (width 0.2) (layer "B.Cu") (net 15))
 (segment (start 77.4475 87.9475) (end 77.25 87.75) (width 0.2) (layer "B.Cu") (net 15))
 (segment (start 77.25 74) (end 74.325 74) (width 0.2) (layer "B.Cu") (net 15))
 (segment (start 77.25 87.75) (end 77.25 74) (width 0.2) (layer "B.Cu") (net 15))
 (segment (start 74.325 74) (end 74.165 74.16) (width 0.2) (layer "B.Cu") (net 15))
 (segment (start 66.8 76.7) (end 58.925 76.7) (width 0.2) (layer "B.Cu") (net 5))
 (segment (start 100.25 64) (end 82.75 64) (width 0.2) (layer "B.Cu") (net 5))
 (segment (start 103.34625 67.09625) (end 100.25 64) (width 0.2) (layer "B.Cu") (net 5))
 (segment (start 103.34625 68.8975) (end 103.34625 67.09625) (width 0.2) (layer "B.Cu") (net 5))
 (segment (start 82.75 64) (end 76.5 70.25) (width 0.2) (layer "B.Cu") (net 5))
 (segment (start 76.5 70.25) (end 73.25 70.25) (width 0.2) (layer "B.Cu") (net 5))
 (segment (start 73.25 70.25) (end 66.8 76.7) (width 0.2) (layer "B.Cu") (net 5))
 (segment (start 76 78.535) (end 74.165 76.7) (width 0.2) (layer "B.Cu") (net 14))
 (segment (start 76 91.25) (end 76 78.535) (width 0.2) (layer "B.Cu") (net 14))
 (segment (start 103.75 88.35125) (end 103.75 93.25) (width 0.2) (layer "B.Cu") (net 14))
 (segment (start 103.34625 87.9475) (end 103.75 88.35125) (width 0.2) (layer "B.Cu") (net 14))
 (segment (start 78 93.25) (end 76 91.25) (width 0.2) (layer "B.Cu") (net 14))
 (segment (start 103.75 93.25) (end 78 93.25) (width 0.2) (layer "B.Cu") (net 14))
 (segment (start 122.39625 68.8975) (end 121.1025 68.8975) (width 0.2) (layer "B.Cu") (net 16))
 (segment (start 121.1025 68.8975) (end 116.75 73.25) (width 0.2) (layer "B.Cu") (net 16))
 (segment (start 116.75 75.5) (end 115.5 76.75) (width 0.2) (layer "B.Cu") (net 16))
 (segment (start 91.5 69.5) (end 88.75 66.75) (width 0.2) (layer "B.Cu") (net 16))
 (segment (start 115.5 76.75) (end 91.5 76.75) (width 0.2) (layer "B.Cu") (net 16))
 (segment (start 78.13 71.62) (end 74.165 71.62) (width 0.2) (layer "B.Cu") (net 16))
 (segment (start 83 66.75) (end 78.13 71.62) (width 0.2) (layer "B.Cu") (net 16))
 (segment (start 91.5 76.75) (end 91.5 69.5) (width 0.2) (layer "B.Cu") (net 16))
 (segment (start 116.75 73.25) (end 116.75 75.5) (width 0.2) (layer "B.Cu") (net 16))
 (segment (start 88.75 66.75) (end 83 66.75) (width 0.2) (layer "B.Cu") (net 16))
 (segment (start 120 99.25) (end 56.5 99.25) (width 0.2) (layer "B.Cu") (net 12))
 (segment (start 122.39625 87.9475) (end 122.39625 96.64625) (width 0.2) (layer "B.Cu") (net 12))
 (segment (start 56.5 99.25) (end 56.5 83) (width 0.2) (layer "B.Cu") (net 12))
 (segment (start 122.5 96.75) (end 120 99.25) (width 0.2) (layer "B.Cu") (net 12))
 (segment (start 56.5 83) (end 58.925 80.575) (width 0.2) (layer "B.Cu") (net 12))
 (segment (start 122.39625 96.64625) (end 122.5 96.75) (width 0.2) (layer "B.Cu") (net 12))
 (segment (start 122.39625 87.9475) (end 122.5 88.05125) (width 0.2) (layer "B.Cu") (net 12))
 (segment (start 58.925 80.575) (end 58.925 79.24) (width 0.2) (layer "B.Cu") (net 12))
 (segment (start 64 93.5) (end 65 94.5) (width 0.2) (layer "F.Cu") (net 1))
 (segment (start 63 93.5) (end 64 93.5) (width 0.2) (layer "F.Cu") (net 1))
 (segment (start 59 96.51) (end 60.101 95.409) (width 0.2) (layer "F.Cu") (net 1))
 (segment (start 65 94.5) (end 66.75 94.5) (width 0.2) (layer "F.Cu") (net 1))
 (segment (start 67.075 93) (end 67 93) (width 0.2) (layer "F.Cu") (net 1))
 (segment (start 59 96.51) (end 59 96.5) (width 0.2) (layer "F.Cu") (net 1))
 (segment (start 61.091 95.409) (end 63 93.5) (width 0.2) (layer "F.Cu") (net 1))
 (segment (start 60.101 95.409) (end 61.091 95.409) (width 0.2) (layer "F.Cu") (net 1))
 (segment (start 67.075 94.175) (end 67.075 93) (width 0.2) (layer "F.Cu") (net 1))
 (segment (start 66.75 94.5) (end 67.075 94.175) (width 0.2) (layer "F.Cu") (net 1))
 (segment (start 65.9207 91.401) (end 66.4207 90.901) (width 0.2) (layer "F.Cu") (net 3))
 (segment (start 69.401 88.5839) (end 70.8339 87.151) (width 0.2) (layer "F.Cu") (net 3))
 (segment (start 73.4161 87.151) (end 73.8171 86.75) (width 0.2) (layer "F.Cu") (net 3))
 (segment (start 60.8161 86.751) (end 59.6661 87.901) (width 0.2) (layer "F.Cu") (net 3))
 (segment (start 74.75 83.5671) (end 74.3339 83.151) (width 0.2) (layer "F.Cu") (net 3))
 (segment (start 68.1661 90.901) (end 69.401 89.6661) (width 0.2) (layer "F.Cu") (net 3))
 (segment (start 74.75 86.2487) (end 74.75 83.5671) (width 0.2) (layer "F.Cu") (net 3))
 (segment (start 61.476 86.751) (end 60.8161 86.751) (width 0.2) (layer "F.Cu") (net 3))
 (segment (start 60.75 93.01) (end 62.359 91.401) (width 0.2) (layer "F.Cu") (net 3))
 (segment (start 61.476 85.774) (end 61.476 86.751) (width 0.2) (layer "F.Cu") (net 3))
 (segment (start 74.3339 83.151) (end 63.099 83.151) (width 0.2) (layer "F.Cu") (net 3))
 (segment (start 62.359 91.401) (end 65.9207 91.401) (width 0.2) (layer "F.Cu") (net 3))
 (segment (start 59.349 87.901) (end 59 88.25) (width 0.2) (layer "F.Cu") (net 3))
 (segment (start 61.5 84.75) (end 61.5 85.75) (width 0.2) (layer "F.Cu") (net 3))
 (segment (start 66.4207 90.901) (end 68.1661 90.901) (width 0.2) (layer "F.Cu") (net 3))
 (segment (start 60.75 93) (end 60.75 93.01) (width 0.2) (layer "F.Cu") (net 3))
 (segment (start 74.2487 86.75) (end 74.75 86.2487) (width 0.2) (layer "F.Cu") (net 3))
 (segment (start 61.5 85.75) (end 61.476 85.774) (width 0.2) (layer "F.Cu") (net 3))
 (segment (start 63.099 83.151) (end 61.5 84.75) (width 0.2) (layer "F.Cu") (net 3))
 (segment (start 70.8339 87.151) (end 73.4161 87.151) (width 0.2) (layer "F.Cu") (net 3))
 (segment (start 59 88.25) (end 59 89.15) (width 0.2) (layer "F.Cu") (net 3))
 (segment (start 73.8171 86.75) (end 74.2487 86.75) (width 0.2) (layer "F.Cu") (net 3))
 (segment (start 69.401 89.6661) (end 69.401 88.5839) (width 0.2) (layer "F.Cu") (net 3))
 (segment (start 59.6661 87.901) (end 59.349 87.901) (width 0.2) (layer "F.Cu") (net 3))
 (segment (start 65.325 96.5) (end 65.325 96.125) (width 0.2) (layer "F.Cu") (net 6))
 (segment (start 65.325 96.125) (end 66.051 95.399) (width 0.2) (layer "F.Cu") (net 6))
 (segment (start 66.051 95.399) (end 72.25 95.399) (width 0.2) (layer "F.Cu") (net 6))
 (segment (start 73.5 94.149) (end 73.5 93) (width 0.2) (layer "F.Cu") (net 6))
 (segment (start 72.25 95.399) (end 73.5 94.149) (width 0.2) (layer "F.Cu") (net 6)))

